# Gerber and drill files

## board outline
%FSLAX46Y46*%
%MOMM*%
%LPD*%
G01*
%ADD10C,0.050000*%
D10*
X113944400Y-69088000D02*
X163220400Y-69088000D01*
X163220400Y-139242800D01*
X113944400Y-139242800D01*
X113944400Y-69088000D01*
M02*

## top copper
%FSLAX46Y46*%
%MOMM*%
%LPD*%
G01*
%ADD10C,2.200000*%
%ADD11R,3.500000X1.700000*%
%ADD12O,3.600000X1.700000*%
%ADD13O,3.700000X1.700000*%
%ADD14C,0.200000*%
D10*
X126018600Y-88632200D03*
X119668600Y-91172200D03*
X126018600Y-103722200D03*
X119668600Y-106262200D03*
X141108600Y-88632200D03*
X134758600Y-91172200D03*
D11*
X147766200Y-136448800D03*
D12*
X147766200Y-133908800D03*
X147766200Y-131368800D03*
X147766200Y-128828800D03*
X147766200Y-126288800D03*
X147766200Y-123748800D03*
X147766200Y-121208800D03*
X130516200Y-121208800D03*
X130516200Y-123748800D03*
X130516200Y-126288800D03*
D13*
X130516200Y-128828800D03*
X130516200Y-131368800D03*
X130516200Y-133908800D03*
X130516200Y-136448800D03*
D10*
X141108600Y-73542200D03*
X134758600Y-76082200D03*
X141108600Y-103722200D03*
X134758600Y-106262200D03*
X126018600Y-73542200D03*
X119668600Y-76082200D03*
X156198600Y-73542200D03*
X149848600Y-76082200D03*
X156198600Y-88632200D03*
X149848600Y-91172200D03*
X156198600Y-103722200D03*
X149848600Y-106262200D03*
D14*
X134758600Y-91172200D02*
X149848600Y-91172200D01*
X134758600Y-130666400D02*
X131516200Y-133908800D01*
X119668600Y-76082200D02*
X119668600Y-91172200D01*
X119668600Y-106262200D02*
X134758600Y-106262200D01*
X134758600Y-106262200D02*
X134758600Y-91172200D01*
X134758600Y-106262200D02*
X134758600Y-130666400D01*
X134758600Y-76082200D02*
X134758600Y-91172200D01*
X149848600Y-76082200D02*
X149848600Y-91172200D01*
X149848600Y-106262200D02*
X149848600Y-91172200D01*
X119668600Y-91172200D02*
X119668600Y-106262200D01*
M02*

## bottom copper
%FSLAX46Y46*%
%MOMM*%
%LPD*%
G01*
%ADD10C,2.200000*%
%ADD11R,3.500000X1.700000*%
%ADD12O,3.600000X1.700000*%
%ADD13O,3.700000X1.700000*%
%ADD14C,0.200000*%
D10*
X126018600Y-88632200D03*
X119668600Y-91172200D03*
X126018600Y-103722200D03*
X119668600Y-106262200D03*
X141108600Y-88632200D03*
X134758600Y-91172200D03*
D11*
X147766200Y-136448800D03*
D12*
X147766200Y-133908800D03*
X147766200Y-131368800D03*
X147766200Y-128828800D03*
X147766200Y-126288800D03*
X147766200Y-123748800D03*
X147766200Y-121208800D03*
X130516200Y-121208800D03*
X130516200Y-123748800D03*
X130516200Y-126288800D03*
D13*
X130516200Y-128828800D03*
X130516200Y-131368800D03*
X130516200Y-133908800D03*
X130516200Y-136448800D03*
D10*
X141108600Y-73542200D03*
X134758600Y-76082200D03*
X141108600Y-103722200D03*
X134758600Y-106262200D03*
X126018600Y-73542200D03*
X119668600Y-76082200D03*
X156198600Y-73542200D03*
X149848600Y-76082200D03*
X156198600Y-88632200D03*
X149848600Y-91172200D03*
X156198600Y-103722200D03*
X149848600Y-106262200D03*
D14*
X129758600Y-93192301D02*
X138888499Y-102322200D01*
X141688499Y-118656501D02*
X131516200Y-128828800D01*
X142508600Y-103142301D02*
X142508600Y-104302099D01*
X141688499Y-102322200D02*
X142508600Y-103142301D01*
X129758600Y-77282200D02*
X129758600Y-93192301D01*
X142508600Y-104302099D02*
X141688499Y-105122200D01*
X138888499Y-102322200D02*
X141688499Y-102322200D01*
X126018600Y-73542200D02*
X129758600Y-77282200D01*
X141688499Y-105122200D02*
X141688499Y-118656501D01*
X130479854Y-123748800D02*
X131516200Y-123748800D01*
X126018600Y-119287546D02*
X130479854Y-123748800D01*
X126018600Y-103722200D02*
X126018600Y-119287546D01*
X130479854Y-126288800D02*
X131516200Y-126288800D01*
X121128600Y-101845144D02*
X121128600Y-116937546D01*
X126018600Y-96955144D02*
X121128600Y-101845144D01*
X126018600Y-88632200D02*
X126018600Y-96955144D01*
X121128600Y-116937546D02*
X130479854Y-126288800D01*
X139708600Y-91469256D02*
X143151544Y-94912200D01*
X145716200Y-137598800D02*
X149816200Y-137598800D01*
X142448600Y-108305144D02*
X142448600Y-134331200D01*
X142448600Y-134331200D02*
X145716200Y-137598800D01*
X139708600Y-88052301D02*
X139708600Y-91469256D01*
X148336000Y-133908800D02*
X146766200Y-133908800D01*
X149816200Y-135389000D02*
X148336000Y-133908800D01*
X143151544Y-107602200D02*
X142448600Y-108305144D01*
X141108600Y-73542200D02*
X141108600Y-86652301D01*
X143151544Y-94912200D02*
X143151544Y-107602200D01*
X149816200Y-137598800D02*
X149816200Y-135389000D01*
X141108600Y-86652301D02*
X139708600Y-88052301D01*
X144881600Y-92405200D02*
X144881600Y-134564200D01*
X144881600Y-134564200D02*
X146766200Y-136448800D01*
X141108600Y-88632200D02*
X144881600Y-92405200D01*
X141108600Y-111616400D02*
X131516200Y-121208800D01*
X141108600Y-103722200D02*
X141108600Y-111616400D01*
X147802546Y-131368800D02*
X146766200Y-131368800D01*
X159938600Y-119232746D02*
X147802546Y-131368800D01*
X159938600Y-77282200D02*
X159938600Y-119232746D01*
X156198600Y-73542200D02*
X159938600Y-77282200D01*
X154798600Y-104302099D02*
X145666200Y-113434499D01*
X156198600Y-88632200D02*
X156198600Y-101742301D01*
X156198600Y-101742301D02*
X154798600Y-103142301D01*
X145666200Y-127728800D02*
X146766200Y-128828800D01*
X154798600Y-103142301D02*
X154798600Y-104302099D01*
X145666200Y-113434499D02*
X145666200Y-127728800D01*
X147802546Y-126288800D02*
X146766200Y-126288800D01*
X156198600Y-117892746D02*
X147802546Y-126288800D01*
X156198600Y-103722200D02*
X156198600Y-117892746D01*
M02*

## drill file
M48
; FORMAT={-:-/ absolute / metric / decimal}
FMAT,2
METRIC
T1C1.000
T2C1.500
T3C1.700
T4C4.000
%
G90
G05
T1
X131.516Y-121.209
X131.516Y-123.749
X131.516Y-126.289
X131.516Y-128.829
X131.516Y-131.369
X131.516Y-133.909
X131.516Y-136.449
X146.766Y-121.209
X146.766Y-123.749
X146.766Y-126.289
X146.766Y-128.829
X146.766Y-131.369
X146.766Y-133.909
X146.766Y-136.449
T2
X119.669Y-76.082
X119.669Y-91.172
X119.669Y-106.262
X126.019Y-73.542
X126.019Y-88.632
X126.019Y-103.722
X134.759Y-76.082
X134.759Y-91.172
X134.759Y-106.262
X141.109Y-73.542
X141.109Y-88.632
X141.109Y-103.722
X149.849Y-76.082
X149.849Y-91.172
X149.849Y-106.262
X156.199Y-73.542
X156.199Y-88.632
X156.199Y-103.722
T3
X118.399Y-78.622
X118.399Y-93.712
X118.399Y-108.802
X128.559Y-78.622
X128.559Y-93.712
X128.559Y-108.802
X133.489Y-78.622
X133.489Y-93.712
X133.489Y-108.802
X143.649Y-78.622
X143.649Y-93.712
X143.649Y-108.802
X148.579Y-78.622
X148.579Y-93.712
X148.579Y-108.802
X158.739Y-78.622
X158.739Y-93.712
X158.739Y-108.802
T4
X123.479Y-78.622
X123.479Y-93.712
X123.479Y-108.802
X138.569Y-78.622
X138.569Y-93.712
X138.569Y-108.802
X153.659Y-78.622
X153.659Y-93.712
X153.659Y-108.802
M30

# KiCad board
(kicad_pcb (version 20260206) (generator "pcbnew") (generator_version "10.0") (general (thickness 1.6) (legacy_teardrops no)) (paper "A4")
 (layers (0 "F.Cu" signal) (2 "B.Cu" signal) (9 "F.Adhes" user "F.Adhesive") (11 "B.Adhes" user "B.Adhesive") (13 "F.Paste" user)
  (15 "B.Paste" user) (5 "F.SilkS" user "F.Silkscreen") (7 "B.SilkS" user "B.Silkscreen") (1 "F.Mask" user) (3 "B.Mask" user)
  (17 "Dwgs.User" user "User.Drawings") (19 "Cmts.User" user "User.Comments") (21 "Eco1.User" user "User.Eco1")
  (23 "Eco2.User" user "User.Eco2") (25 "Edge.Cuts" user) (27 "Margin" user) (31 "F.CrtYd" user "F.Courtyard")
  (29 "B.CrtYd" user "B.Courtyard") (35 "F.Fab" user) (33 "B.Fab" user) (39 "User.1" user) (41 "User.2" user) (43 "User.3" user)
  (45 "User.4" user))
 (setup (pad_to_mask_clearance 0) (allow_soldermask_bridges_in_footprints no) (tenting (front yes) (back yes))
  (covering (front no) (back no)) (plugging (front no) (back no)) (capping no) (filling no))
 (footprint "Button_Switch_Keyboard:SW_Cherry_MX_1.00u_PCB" (layer "F.Cu") (at 126.0186 88.6322)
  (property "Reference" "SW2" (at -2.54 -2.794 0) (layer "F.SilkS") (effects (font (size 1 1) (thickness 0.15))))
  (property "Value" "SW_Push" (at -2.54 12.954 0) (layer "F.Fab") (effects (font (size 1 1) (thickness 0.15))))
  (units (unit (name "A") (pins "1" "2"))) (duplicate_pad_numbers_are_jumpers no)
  (pad "" np_thru_hole circle (at -7.62 5.08) (size 1.7 1.7) (drill 1.7) (layers "*.Cu" "*.Mask"))
  (pad "" np_thru_hole circle (at -2.54 5.08) (size 4 4) (drill 4) (layers "*.Cu" "*.Mask"))
  (pad "" np_thru_hole circle (at 2.54 5.08) (size 1.7 1.7) (drill 1.7) (layers "*.Cu" "*.Mask"))
  (pad "1" thru_hole circle (at 0 0) (size 2.2 2.2) (drill 1.5) (layers "*.Cu" "*.Mask") (remove_unused_layers no)
   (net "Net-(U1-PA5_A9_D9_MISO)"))
  (pad "2" thru_hole circle (at -6.35 2.54) (size 2.2 2.2) (drill 1.5) (layers "*.Cu" "*.Mask") (remove_unused_layers no) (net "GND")))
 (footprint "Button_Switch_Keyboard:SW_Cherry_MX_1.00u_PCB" (layer "F.Cu") (at 126.0186 103.7222)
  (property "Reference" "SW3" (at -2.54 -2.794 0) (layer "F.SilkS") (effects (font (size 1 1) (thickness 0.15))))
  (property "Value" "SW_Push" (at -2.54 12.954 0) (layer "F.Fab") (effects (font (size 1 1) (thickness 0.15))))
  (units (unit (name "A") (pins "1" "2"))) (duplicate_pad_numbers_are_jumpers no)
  (pad "" np_thru_hole circle (at -7.62 5.08) (size 1.7 1.7) (drill 1.7) (layers "*.Cu" "*.Mask"))
  (pad "" np_thru_hole circle (at -2.54 5.08) (size 4 4) (drill 4) (layers "*.Cu" "*.Mask"))
  (pad "" np_thru_hole circle (at 2.54 5.08) (size 1.7 1.7) (drill 1.7) (layers "*.Cu" "*.Mask"))
  (pad "1" thru_hole circle (at 0 0) (size 2.2 2.2) (drill 1.5) (layers "*.Cu" "*.Mask") (remove_unused_layers no)
   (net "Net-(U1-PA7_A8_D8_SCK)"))
  (pad "2" thru_hole circle (at -6.35 2.54) (size 2.2 2.2) (drill 1.5) (layers "*.Cu" "*.Mask") (remove_unused_layers no) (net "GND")))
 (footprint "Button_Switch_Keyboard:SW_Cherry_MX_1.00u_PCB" (layer "F.Cu") (at 141.1086 88.6322)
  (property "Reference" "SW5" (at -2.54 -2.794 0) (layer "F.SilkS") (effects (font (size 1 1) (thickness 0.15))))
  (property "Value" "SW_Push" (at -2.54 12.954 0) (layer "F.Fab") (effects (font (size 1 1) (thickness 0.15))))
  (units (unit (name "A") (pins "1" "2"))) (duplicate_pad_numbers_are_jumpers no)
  (pad "" np_thru_hole circle (at -7.62 5.08) (size 1.7 1.7) (drill 1.7) (layers "*.Cu" "*.Mask"))
  (pad "" np_thru_hole circle (at -2.54 5.08) (size 4 4) (drill 4) (layers "*.Cu" "*.Mask"))
  (pad "" np_thru_hole circle (at 2.54 5.08) (size 1.7 1.7) (drill 1.7) (layers "*.Cu" "*.Mask"))
  (pad "1" thru_hole circle (at 0 0) (size 2.2 2.2) (drill 1.5) (layers "*.Cu" "*.Mask") (remove_unused_layers no)
   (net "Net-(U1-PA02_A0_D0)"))
  (pad "2" thru_hole circle (at -6.35 2.54) (size 2.2 2.2) (drill 1.5) (layers "*.Cu" "*.Mask") (remove_unused_layers no) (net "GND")))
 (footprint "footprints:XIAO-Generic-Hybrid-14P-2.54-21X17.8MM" (layer "F.Cu") (at 139.1412 128.8288 180)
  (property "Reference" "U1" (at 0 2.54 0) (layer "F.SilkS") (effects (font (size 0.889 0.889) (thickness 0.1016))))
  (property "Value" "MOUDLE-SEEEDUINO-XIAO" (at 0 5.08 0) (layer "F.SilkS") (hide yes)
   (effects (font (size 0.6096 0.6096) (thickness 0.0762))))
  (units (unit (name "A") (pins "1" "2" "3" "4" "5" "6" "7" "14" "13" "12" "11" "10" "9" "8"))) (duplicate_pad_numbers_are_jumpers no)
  (pad "1" thru_hole rect (at -7.625 -7.62 180) (size 3.5 1.7) (drill 1 (offset -1 0)) (layers "*.Cu" "*.Mask") (remove_unused_layers no)
   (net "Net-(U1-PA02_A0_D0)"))
  (pad "2" thru_hole oval (at -7.625 -5.08 180) (size 3.6 1.7) (drill 1 (offset -1 0)) (layers "*.Cu" "*.Mask") (remove_unused_layers no)
   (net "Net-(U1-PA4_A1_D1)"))
  (pad "3" thru_hole oval (at -7.625 -2.54 180) (size 3.6 1.7) (drill 1 (offset -1 0)) (layers "*.Cu" "*.Mask") (remove_unused_layers no)
   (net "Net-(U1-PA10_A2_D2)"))
  (pad "4" thru_hole oval (at -7.625 0 180) (size 3.6 1.7) (drill 1 (offset -1 0)) (layers "*.Cu" "*.Mask") (remove_unused_layers no)
   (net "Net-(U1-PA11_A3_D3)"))
  (pad "5" thru_hole oval (at -7.625 2.54 180) (size 3.6 1.7) (drill 1 (offset -1 0)) (layers "*.Cu" "*.Mask") (remove_unused_layers no)
   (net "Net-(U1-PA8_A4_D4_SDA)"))
  (pad "6" thru_hole oval (at -7.625 5.08) (size 3.6 1.7) (drill 1 (offset 1 0)) (layers "*.Cu" "*.Mask") (remove_unused_layers no)
   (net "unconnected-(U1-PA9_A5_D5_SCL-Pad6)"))
  (pad "7" thru_hole oval (at -7.625 7.62 180) (size 3.6 1.7) (drill 1 (offset -1 0)) (layers "*.Cu" "*.Mask") (remove_unused_layers no)
   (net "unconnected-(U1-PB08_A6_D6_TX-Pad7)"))
  (pad "8" thru_hole oval (at 7.625 7.62 180) (size 3.6 1.7) (drill 1 (offset 1 0)) (layers "*.Cu" "*.Mask") (remove_unused_layers no)
   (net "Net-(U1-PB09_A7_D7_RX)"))
  (pad "9" thru_hole oval (at 7.625 5.08 180) (size 3.6 1.7) (drill 1 (offset 1 0)) (layers "*.Cu" "*.Mask") (remove_unused_layers no)
   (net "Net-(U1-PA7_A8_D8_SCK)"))
  (pad "10" thru_hole oval (at 7.625 2.54 180) (size 3.6 1.7) (drill 1 (offset 1 0)) (layers "*.Cu" "*.Mask") (remove_unused_layers no)
   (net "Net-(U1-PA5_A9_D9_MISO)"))
  (pad "11" thru_hole oval (at 7.625 0 180) (size 3.7 1.7) (drill 1 (offset 1 0)) (layers "*.Cu" "*.Mask") (remove_unused_layers no)
   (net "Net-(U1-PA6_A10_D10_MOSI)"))
  (pad "12" thru_hole oval (at 7.625 -2.54 180) (size 3.7 1.7) (drill 1 (offset 1 0)) (layers "*.Cu" "*.Mask") (remove_unused_layers no)
   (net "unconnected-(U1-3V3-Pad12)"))
  (pad "13" thru_hole oval (at 7.625 -5.08 180) (size 3.7 1.7) (drill 1 (offset 1 0)) (layers "*.Cu" "*.Mask") (remove_unused_layers no)
   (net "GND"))
  (pad "14" thru_hole oval (at 7.625 -7.62 180) (size 3.7 1.7) (drill 1 (offset 1 0)) (layers "*.Cu" "*.Mask") (remove_unused_layers no)
   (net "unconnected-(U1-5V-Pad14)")))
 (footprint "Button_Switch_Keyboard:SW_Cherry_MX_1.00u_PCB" (layer "F.Cu") (at 141.1086 73.5422)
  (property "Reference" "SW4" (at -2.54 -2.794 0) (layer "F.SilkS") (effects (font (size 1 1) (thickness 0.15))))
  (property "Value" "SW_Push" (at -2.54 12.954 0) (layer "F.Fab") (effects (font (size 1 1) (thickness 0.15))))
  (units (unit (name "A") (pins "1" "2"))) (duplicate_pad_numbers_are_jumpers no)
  (pad "" np_thru_hole circle (at -7.62 5.08) (size 1.7 1.7) (drill 1.7) (layers "*.Cu" "*.Mask"))
  (pad "" np_thru_hole circle (at -2.54 5.08) (size 4 4) (drill 4) (layers "*.Cu" "*.Mask"))
  (pad "" np_thru_hole circle (at 2.54 5.08) (size 1.7 1.7) (drill 1.7) (layers "*.Cu" "*.Mask"))
  (pad "1" thru_hole circle (at 0 0) (size 2.2 2.2) (drill 1.5) (layers "*.Cu" "*.Mask") (remove_unused_layers no)
   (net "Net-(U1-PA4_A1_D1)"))
  (pad "2" thru_hole circle (at -6.35 2.54) (size 2.2 2.2) (drill 1.5) (layers "*.Cu" "*.Mask") (remove_unused_layers no) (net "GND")))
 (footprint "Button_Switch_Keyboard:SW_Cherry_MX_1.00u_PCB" (layer "F.Cu") (at 141.1086 103.7222)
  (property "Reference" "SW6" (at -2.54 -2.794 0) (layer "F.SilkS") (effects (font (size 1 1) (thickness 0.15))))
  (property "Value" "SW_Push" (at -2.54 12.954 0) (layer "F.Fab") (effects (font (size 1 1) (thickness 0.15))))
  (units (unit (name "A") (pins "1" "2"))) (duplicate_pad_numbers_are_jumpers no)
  (pad "" np_thru_hole circle (at -7.62 5.08) (size 1.7 1.7) (drill 1.7) (layers "*.Cu" "*.Mask"))
  (pad "" np_thru_hole circle (at -2.54 5.08) (size 4 4) (drill 4) (layers "*.Cu" "*.Mask"))
  (pad "" np_thru_hole circle (at 2.54 5.08) (size 1.7 1.7) (drill 1.7) (layers "*.Cu" "*.Mask"))
  (pad "1" thru_hole circle (at 0 0) (size 2.2 2.2) (drill 1.5) (layers "*.Cu" "*.Mask") (remove_unused_layers no)
   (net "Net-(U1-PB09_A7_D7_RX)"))
  (pad "2" thru_hole circle (at -6.35 2.54) (size 2.2 2.2) (drill 1.5) (layers "*.Cu" "*.Mask") (remove_unused_layers no) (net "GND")))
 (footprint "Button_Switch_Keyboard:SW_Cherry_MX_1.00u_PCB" (layer "F.Cu") (at 126.0186 73.5422)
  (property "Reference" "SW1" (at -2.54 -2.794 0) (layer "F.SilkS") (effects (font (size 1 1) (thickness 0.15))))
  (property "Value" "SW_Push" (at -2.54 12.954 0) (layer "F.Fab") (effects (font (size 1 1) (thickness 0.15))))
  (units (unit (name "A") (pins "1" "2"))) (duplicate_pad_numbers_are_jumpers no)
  (pad "" np_thru_hole circle (at -7.62 5.08) (size 1.7 1.7) (drill 1.7) (layers "*.Cu" "*.Mask"))
  (pad "" np_thru_hole circle (at -2.54 5.08) (size 4 4) (drill 4) (layers "*.Cu" "*.Mask"))
  (pad "" np_thru_hole circle (at 2.54 5.08) (size 1.7 1.7) (drill 1.7) (layers "*.Cu" "*.Mask"))
  (pad "1" thru_hole circle (at 0 0) (size 2.2 2.2) (drill 1.5) (layers "*.Cu" "*.Mask") (remove_unused_layers no)
   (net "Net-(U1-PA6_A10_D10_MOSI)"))
  (pad "2" thru_hole circle (at -6.35 2.54) (size 2.2 2.2) (drill 1.5) (layers "*.Cu" "*.Mask") (remove_unused_layers no) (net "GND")))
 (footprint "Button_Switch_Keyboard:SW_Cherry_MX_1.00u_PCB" (layer "F.Cu") (at 156.1986 73.5422)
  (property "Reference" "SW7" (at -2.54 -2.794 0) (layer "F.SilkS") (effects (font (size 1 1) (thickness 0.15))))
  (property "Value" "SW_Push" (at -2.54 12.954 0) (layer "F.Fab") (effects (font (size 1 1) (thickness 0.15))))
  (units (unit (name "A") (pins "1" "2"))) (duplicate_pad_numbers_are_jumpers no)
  (pad "" np_thru_hole circle (at -7.62 5.08) (size 1.7 1.7) (drill 1.7) (layers "*.Cu" "*.Mask"))
  (pad "" np_thru_hole circle (at -2.54 5.08) (size 4 4) (drill 4) (layers "*.Cu" "*.Mask"))
  (pad "" np_thru_hole circle (at 2.54 5.08) (size 1.7 1.7) (drill 1.7) (layers "*.Cu" "*.Mask"))
  (pad "1" thru_hole circle (at 0 0) (size 2.2 2.2) (drill 1.5) (layers "*.Cu" "*.Mask") (remove_unused_layers no)
   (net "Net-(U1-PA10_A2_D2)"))
  (pad "2" thru_hole circle (at -6.35 2.54) (size 2.2 2.2) (drill 1.5) (layers "*.Cu" "*.Mask") (remove_unused_layers no) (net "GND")))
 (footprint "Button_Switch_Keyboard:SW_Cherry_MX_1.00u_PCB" (layer "F.Cu") (at 156.1986 88.6322)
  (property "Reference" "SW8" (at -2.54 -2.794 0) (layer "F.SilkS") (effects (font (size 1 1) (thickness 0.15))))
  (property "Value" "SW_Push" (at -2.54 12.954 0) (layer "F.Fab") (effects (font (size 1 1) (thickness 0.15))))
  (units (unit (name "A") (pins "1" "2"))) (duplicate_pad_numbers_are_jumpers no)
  (pad "" np_thru_hole circle (at -7.62 5.08) (size 1.7 1.7) (drill 1.7) (layers "*.Cu" "*.Mask"))
  (pad "" np_thru_hole circle (at -2.54 5.08) (size 4 4) (drill 4) (layers "*.Cu" "*.Mask"))
  (pad "" np_thru_hole circle (at 2.54 5.08) (size 1.7 1.7) (drill 1.7) (layers "*.Cu" "*.Mask"))
  (pad "1" thru_hole circle (at 0 0) (size 2.2 2.2) (drill 1.5) (layers "*.Cu" "*.Mask") (remove_unused_layers no)
   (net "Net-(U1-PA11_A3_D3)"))
  (pad "2" thru_hole circle (at -6.35 2.54) (size 2.2 2.2) (drill 1.5) (layers "*.Cu" "*.Mask") (remove_unused_layers no) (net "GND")))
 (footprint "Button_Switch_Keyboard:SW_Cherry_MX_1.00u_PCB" (layer "F.Cu") (at 156.1986 103.7222)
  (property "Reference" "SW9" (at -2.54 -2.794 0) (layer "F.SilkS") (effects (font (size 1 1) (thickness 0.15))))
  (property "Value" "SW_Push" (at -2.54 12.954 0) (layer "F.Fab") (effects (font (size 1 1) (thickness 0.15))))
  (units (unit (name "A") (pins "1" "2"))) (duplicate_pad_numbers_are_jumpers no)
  (pad "" np_thru_hole circle (at -7.62 5.08) (size 1.7 1.7) (drill 1.7) (layers "*.Cu" "*.Mask"))
  (pad "" np_thru_hole circle (at -2.54 5.08) (size 4 4) (drill 4) (layers "*.Cu" "*.Mask"))
  (pad "" np_thru_hole circle (at 2.54 5.08) (size 1.7 1.7) (drill 1.7) (layers "*.Cu" "*.Mask"))
  (pad "1" thru_hole circle (at 0 0) (size 2.2 2.2) (drill 1.5) (layers "*.Cu" "*.Mask") (remove_unused_layers no)
   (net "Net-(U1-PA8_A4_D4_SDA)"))
  (pad "2" thru_hole circle (at -6.35 2.54) (size 2.2 2.2) (drill 1.5) (layers "*.Cu" "*.Mask") (remove_unused_layers no) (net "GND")))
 (gr_rect (start 113.9444 69.088) (end 163.2204 139.2428) (stroke (width 0.05) (type default)) (fill no) (layer "Edge.Cuts"))
 (segment (start 129.7586 93.192301) (end 138.888499 102.3222) (width 0.2) (layer "B.Cu") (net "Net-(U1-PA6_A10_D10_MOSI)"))
 (segment (start 141.688499 118.656501) (end 131.5162 128.8288) (width 0.2) (layer "B.Cu") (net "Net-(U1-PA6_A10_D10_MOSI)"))
 (segment (start 142.5086 103.142301) (end 142.5086 104.302099) (width 0.2) (layer "B.Cu") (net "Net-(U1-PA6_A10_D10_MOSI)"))
 (segment (start 141.688499 102.3222) (end 142.5086 103.142301) (width 0.2) (layer "B.Cu") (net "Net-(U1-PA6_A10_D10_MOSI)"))
 (segment (start 129.7586 77.2822) (end 129.7586 93.192301) (width 0.2) (layer "B.Cu") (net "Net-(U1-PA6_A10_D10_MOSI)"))
 (segment (start 142.5086 104.302099) (end 141.688499 105.1222) (width 0.2) (layer "B.Cu") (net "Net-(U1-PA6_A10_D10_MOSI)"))
 (segment (start 138.888499 102.3222) (end 141.688499 102.3222) (width 0.2) (layer "B.Cu") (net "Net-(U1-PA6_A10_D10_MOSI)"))
 (segment (start 126.0186 73.5422) (end 129.7586 77.2822) (width 0.2) (layer "B.Cu") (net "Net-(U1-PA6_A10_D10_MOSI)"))
 (segment (start 141.688499 105.1222) (end 141.688499 118.656501) (width 0.2) (layer "B.Cu") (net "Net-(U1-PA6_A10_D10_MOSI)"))
 (segment (start 134.7586 91.1722) (end 149.8486 91.1722) (width 0.2) (layer "F.Cu") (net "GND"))
 (segment (start 134.7586 130.6664) (end 131.5162 133.9088) (width 0.2) (layer "F.Cu") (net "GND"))
 (segment (start 119.6686 76.0822) (end 119.6686 91.1722) (width 0.2) (layer "F.Cu") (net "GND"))
 (segment (start 119.6686 106.2622) (end 134.7586 106.2622) (width 0.2) (layer "F.Cu") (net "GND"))
 (segment (start 134.7586 106.2622) (end 134.7586 91.1722) (width 0.2) (layer "F.Cu") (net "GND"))
 (segment (start 134.7586 106.2622) (end 134.7586 130.6664) (width 0.2) (layer "F.Cu") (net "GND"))
 (segment (start 134.7586 76.0822) (end 134.7586 91.1722) (width 0.2) (layer "F.Cu") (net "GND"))
 (segment (start 149.8486 76.0822) (end 149.8486 91.1722) (width 0.2) (layer "F.Cu") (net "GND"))
 (segment (start 149.8486 106.2622) (end 149.8486 91.1722) (width 0.2) (layer "F.Cu") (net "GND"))
 (segment (start 119.6686 91.1722) (end 119.6686 106.2622) (width 0.2) (layer "F.Cu") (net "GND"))
 (segment (start 130.479854 123.7488) (end 131.5162 123.7488) (width 0.2) (layer "B.Cu") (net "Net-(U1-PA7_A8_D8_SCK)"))
 (segment (start 126.0186 119.287546) (end 130.479854 123.7488) (width 0.2) (layer "B.Cu") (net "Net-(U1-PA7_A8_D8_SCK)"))
 (segment (start 126.0186 103.7222) (end 126.0186 119.287546) (width 0.2) (layer "B.Cu") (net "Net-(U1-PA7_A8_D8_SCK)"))
 (segment (start 130.479854 126.2888) (end 131.5162 126.2888) (width 0.2) (layer "B.Cu") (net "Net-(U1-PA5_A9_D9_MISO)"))
 (segment (start 121.1286 101.845144) (end 121.1286 116.937546) (width 0.2) (layer "B.Cu") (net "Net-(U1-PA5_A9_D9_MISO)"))
 (segment (start 126.0186 96.955144) (end 121.1286 101.845144) (width 0.2) (layer "B.Cu") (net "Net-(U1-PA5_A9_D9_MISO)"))
 (segment (start 126.0186 88.6322) (end 126.0186 96.955144) (width 0.2) (layer "B.Cu") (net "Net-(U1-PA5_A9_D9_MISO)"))
 (segment (start 121.1286 116.937546) (end 130.479854 126.2888) (width 0.2) (layer "B.Cu") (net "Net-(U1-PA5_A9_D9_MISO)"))
 (segment (start 139.7086 91.469256) (end 143.151544 94.9122) (width 0.2) (layer "B.Cu") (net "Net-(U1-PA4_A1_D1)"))
 (segment (start 145.7162 137.5988) (end 149.8162 137.5988) (width 0.2) (layer "B.Cu") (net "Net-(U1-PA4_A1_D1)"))
 (segment (start 142.4486 108.305144) (end 142.4486 134.3312) (width 0.2) (layer "B.Cu") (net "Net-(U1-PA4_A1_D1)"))
 (segment (start 142.4486 134.3312) (end 145.7162 137.5988) (width 0.2) (layer "B.Cu") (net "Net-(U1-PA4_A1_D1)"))
 (segment (start 139.7086 88.052301) (end 139.7086 91.469256) (width 0.2) (layer "B.Cu") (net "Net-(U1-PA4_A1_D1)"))
 (segment (start 148.336 133.9088) (end 146.7662 133.9088) (width 0.2) (layer "B.Cu") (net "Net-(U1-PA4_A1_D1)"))
 (segment (start 149.8162 135.389) (end 148.336 133.9088) (width 0.2) (layer "B.Cu") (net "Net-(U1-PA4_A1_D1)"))
 (segment (start 143.151544 107.6022) (end 142.4486 108.305144) (width 0.2) (layer "B.Cu") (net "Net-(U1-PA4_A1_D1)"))
 (segment (start 141.1086 73.5422) (end 141.1086 86.652301) (width 0.2) (layer "B.Cu") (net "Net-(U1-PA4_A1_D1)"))
 (segment (start 143.151544 94.9122) (end 143.151544 107.6022) (width 0.2) (layer "B.Cu") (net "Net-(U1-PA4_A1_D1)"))
 (segment (start 149.8162 137.5988) (end 149.8162 135.389) (width 0.2) (layer "B.Cu") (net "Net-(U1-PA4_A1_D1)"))
 (segment (start 141.1086 86.652301) (end 139.7086 88.052301) (width 0.2) (layer "B.Cu") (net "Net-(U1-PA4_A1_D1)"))
 (segment (start 144.8816 92.4052) (end 144.8816 134.5642) (width 0.2) (layer "B.Cu") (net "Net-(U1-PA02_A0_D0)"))
 (segment (start 144.8816 134.5642) (end 146.7662 136.4488) (width 0.2) (layer "B.Cu") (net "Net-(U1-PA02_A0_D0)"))
 (segment (start 141.1086 88.6322) (end 144.8816 92.4052) (width 0.2) (layer "B.Cu") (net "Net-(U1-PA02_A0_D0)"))
 (segment (start 141.1086 111.6164) (end 131.5162 121.2088) (width 0.2) (layer "B.Cu") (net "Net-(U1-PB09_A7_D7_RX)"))
 (segment (start 141.1086 103.7222) (end 141.1086 111.6164) (width 0.2) (layer "B.Cu") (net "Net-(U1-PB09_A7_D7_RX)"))
 (segment (start 147.802546 131.3688) (end 146.7662 131.3688) (width 0.2) (layer "B.Cu") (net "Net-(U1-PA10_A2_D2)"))
 (segment (start 159.9386 119.232746) (end 147.802546 131.3688) (width 0.2) (layer "B.Cu") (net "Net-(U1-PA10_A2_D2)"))
 (segment (start 159.9386 77.2822) (end 159.9386 119.232746) (width 0.2) (layer "B.Cu") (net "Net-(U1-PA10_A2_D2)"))
 (segment (start 156.1986 73.5422) (end 159.9386 77.2822) (width 0.2) (layer "B.Cu") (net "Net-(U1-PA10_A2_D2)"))
 (segment (start 154.7986 104.302099) (end 145.6662 113.434499) (width 0.2) (layer "B.Cu") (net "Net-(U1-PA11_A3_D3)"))
 (segment (start 156.1986 88.6322) (end 156.1986 101.742301) (width 0.2) (layer "B.Cu") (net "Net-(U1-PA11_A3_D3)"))
 (segment (start 156.1986 101.742301) (end 154.7986 103.142301) (width 0.2) (layer "B.Cu") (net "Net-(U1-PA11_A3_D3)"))
 (segment (start 145.6662 127.7288) (end 146.7662 128.8288) (width 0.2) (layer "B.Cu") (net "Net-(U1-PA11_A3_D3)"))
 (segment (start 154.7986 103.142301) (end 154.7986 104.302099) (width 0.2) (layer "B.Cu") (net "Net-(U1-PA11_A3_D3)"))
 (segment (start 145.6662 113.434499) (end 145.6662 127.7288) (width 0.2) (layer "B.Cu") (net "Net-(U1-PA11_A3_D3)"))
 (segment (start 147.802546 126.2888) (end 146.7662 126.2888) (width 0.2) (layer "B.Cu") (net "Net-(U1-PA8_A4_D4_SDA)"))
 (segment (start 156.1986 117.892746) (end 147.802546 126.2888) (width 0.2) (layer "B.Cu") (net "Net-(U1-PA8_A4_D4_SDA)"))
 (segment (start 156.1986 103.7222) (end 156.1986 117.892746) (width 0.2) (layer "B.Cu") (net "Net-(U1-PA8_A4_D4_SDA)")))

